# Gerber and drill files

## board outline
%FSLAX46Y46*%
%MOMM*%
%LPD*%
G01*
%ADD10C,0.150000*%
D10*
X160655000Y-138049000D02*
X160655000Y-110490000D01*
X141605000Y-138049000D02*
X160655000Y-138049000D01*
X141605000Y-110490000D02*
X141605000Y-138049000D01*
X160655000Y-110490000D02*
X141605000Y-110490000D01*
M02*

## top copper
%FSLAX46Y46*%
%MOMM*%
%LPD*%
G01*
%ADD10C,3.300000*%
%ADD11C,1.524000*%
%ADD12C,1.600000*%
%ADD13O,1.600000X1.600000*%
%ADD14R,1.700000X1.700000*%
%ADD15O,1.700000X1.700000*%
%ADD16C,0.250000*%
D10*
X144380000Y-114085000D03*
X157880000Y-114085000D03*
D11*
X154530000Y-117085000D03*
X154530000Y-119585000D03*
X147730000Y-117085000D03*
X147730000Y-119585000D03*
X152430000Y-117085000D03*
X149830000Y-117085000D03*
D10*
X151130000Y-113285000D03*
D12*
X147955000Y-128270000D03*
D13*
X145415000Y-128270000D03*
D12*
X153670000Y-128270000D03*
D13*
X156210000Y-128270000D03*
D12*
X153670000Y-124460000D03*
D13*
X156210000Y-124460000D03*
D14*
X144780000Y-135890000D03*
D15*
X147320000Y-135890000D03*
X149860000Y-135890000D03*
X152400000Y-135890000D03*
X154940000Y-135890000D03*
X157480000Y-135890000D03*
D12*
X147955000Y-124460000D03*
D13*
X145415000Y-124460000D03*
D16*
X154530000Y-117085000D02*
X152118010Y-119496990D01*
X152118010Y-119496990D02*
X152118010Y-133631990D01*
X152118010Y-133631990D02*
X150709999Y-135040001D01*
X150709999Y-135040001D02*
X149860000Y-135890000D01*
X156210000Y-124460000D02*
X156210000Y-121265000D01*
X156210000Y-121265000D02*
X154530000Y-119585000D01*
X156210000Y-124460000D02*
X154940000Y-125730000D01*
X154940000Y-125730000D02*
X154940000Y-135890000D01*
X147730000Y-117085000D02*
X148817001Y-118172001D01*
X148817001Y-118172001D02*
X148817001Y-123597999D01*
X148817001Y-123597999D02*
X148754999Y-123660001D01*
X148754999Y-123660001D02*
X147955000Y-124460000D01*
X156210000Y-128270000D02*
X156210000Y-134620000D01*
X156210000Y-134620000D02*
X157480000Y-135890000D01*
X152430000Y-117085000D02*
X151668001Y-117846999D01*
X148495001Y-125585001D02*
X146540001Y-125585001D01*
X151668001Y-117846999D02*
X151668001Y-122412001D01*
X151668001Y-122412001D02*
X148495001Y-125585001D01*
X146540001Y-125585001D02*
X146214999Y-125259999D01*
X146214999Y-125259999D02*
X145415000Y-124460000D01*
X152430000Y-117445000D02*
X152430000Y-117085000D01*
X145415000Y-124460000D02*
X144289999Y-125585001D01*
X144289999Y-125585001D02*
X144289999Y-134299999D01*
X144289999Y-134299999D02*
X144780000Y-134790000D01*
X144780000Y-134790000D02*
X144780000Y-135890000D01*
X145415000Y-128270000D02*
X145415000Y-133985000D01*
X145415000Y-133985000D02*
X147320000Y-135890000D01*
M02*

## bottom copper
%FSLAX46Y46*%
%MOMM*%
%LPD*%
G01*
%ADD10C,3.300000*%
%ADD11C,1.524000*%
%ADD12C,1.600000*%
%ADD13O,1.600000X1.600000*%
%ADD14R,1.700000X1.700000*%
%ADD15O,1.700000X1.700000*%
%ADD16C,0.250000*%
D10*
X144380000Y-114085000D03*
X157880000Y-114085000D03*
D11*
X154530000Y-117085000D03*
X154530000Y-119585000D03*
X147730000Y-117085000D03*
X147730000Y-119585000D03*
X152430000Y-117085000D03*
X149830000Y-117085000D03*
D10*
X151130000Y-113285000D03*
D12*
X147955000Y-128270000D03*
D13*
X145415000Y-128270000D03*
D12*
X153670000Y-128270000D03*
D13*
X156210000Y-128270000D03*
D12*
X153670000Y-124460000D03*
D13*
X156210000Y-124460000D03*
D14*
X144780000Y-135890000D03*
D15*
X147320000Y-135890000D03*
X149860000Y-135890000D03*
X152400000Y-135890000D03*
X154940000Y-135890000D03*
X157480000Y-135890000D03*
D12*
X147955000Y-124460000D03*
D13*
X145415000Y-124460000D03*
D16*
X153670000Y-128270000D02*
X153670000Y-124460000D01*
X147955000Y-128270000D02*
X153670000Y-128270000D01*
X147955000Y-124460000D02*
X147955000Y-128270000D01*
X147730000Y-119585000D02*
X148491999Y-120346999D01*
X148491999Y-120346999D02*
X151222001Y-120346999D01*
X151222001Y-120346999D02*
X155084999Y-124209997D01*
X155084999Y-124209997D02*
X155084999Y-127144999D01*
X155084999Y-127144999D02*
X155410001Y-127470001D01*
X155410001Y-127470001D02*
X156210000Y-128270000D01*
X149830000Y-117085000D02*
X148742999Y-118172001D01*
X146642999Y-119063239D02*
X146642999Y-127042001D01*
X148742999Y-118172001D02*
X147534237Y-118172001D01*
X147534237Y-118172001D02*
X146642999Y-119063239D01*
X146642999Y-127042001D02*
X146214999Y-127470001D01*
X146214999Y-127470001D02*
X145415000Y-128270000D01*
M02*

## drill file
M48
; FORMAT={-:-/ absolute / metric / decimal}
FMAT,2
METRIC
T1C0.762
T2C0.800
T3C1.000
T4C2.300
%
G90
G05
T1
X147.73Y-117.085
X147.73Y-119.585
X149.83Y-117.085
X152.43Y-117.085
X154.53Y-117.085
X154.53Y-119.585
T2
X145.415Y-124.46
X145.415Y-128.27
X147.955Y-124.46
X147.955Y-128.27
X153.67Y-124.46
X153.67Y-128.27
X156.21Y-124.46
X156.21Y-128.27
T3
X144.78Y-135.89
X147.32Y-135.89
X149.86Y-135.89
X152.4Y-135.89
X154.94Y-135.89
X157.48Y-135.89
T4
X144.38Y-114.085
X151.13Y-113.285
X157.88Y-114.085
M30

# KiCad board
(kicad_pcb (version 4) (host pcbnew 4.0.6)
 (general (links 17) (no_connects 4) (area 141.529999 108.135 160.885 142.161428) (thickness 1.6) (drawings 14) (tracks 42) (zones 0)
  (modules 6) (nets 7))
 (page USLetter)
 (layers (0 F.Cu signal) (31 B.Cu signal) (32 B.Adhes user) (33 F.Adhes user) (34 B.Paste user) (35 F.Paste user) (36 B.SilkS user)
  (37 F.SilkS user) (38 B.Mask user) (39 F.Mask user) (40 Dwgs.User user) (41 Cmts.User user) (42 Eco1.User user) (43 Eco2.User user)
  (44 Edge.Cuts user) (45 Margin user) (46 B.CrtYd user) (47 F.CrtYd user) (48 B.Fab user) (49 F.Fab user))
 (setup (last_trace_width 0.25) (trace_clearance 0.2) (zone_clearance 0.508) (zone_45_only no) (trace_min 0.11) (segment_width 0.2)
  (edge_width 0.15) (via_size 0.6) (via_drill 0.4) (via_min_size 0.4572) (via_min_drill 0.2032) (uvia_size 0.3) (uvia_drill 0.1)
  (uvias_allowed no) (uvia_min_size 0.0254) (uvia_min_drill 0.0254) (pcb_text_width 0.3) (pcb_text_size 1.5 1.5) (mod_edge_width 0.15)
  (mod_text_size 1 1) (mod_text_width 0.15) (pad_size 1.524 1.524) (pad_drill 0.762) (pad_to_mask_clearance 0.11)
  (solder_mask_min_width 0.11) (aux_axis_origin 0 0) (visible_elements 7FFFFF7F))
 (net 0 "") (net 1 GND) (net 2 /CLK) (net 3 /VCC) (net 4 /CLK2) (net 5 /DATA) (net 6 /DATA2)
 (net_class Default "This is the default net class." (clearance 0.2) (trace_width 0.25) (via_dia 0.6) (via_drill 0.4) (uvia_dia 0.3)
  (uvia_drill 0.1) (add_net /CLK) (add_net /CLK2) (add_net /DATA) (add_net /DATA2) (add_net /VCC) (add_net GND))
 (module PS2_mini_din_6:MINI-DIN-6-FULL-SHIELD (layer F.Cu) (at 151.13 108.585)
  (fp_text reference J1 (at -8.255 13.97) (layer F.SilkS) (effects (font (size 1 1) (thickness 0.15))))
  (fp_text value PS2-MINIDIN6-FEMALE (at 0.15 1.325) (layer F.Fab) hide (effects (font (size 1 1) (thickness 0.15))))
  (pad 7 thru_hole circle (at -6.75 5.5) (size 3.3 3.3) (drill 2.3) (layers *.Cu *.Mask) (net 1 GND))
  (pad 7 thru_hole circle (at 6.75 5.5) (size 3.3 3.3) (drill 2.3) (layers *.Cu *.Mask) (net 1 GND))
  (pad 3 thru_hole circle (at 3.4 8.5) (size 1.524 1.524) (drill 0.762) (layers *.Cu *.Mask) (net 1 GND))
  (pad 5 thru_hole circle (at 3.4 11) (size 1.524 1.524) (drill 0.762) (layers *.Cu *.Mask) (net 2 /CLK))
  (pad 4 thru_hole circle (at -3.4 8.5) (size 1.524 1.524) (drill 0.762) (layers *.Cu *.Mask) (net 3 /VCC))
  (pad 6 thru_hole circle (at -3.4 11) (size 1.524 1.524) (drill 0.762) (layers *.Cu *.Mask) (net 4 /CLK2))
  (pad 1 thru_hole circle (at 1.3 8.5) (size 1.524 1.524) (drill 0.762) (layers *.Cu *.Mask) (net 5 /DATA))
  (pad 2 thru_hole circle (at -1.3 8.5) (size 1.524 1.524) (drill 0.762) (layers *.Cu *.Mask) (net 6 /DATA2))
  (pad 7 thru_hole circle (at 0 4.7) (size 3.3 3.3) (drill 2.3) (layers *.Cu *.Mask) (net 1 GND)))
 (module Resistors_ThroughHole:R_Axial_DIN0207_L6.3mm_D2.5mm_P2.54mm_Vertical (layer F.Cu) (at 147.955 128.27 180)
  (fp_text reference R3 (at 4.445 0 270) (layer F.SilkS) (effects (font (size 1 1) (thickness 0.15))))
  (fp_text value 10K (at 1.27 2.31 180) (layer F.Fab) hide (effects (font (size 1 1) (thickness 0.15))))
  (pad 1 thru_hole circle (at 0 0 180) (size 1.6 1.6) (drill 0.8) (layers *.Cu *.Mask) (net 3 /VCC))
  (pad 2 thru_hole oval (at 2.54 0 180) (size 1.6 1.6) (drill 0.8) (layers *.Cu *.Mask) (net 6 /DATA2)))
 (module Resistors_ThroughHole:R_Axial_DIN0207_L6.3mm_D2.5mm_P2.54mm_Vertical (layer F.Cu) (at 153.67 128.27)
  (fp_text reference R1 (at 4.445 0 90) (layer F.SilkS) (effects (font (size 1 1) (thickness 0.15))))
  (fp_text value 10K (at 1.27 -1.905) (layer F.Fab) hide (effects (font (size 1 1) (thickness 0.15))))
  (pad 1 thru_hole circle (at 0 0) (size 1.6 1.6) (drill 0.8) (layers *.Cu *.Mask) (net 3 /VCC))
  (pad 2 thru_hole oval (at 2.54 0) (size 1.6 1.6) (drill 0.8) (layers *.Cu *.Mask) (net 4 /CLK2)))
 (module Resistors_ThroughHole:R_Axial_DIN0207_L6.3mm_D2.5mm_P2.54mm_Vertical (layer F.Cu) (at 153.67 124.46)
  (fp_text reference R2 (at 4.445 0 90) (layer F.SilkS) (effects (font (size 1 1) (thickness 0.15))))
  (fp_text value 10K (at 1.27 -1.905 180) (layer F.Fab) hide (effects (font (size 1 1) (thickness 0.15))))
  (pad 1 thru_hole circle (at 0 0) (size 1.6 1.6) (drill 0.8) (layers *.Cu *.Mask) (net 3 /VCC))
  (pad 2 thru_hole oval (at 2.54 0) (size 1.6 1.6) (drill 0.8) (layers *.Cu *.Mask) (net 2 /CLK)))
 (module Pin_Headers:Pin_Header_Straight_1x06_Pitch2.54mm (layer F.Cu) (at 144.78 135.89 90)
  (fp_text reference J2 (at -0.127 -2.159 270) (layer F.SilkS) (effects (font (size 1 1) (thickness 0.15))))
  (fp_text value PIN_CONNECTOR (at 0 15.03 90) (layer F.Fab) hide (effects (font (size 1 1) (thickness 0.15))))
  (pad 1 thru_hole rect (at 0 0 90) (size 1.7 1.7) (drill 1) (layers *.Cu *.Mask) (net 5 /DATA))
  (pad 2 thru_hole oval (at 0 2.54 90) (size 1.7 1.7) (drill 1) (layers *.Cu *.Mask) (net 6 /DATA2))
  (pad 3 thru_hole oval (at 0 5.08 90) (size 1.7 1.7) (drill 1) (layers *.Cu *.Mask) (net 1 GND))
  (pad 4 thru_hole oval (at 0 7.62 90) (size 1.7 1.7) (drill 1) (layers *.Cu *.Mask) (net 3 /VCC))
  (pad 5 thru_hole oval (at 0 10.16 90) (size 1.7 1.7) (drill 1) (layers *.Cu *.Mask) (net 2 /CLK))
  (pad 6 thru_hole oval (at 0 12.7 90) (size 1.7 1.7) (drill 1) (layers *.Cu *.Mask) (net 4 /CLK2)))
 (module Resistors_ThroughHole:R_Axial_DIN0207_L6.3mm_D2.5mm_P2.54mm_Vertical (layer F.Cu) (at 147.955 124.46 180)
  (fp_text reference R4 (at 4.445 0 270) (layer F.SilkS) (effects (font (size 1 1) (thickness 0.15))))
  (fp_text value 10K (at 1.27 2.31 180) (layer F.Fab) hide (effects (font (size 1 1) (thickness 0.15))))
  (pad 1 thru_hole circle (at 0 0 180) (size 1.6 1.6) (drill 0.8) (layers *.Cu *.Mask) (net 3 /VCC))
  (pad 2 thru_hole oval (at 2.54 0 180) (size 1.6 1.6) (drill 0.8) (layers *.Cu *.Mask) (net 5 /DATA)))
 (gr_line (start 160.655 138.049) (end 160.655 110.49) (layer Edge.Cuts) (width 0.15))
 (gr_line (start 141.605 138.049) (end 160.655 138.049) (layer Edge.Cuts) (width 0.15))
 (gr_line (start 141.605 110.49) (end 141.605 138.049) (layer Edge.Cuts) (width 0.15))
 (gr_line (start 160.655 110.49) (end 141.605 110.49) (layer Edge.Cuts) (width 0.15))
 (segment (start 154.53 117.085) (end 152.11801 119.49699) (width 0.25) (layer F.Cu) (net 1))
 (segment (start 152.11801 119.49699) (end 152.11801 133.63199) (width 0.25) (layer F.Cu) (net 1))
 (segment (start 152.11801 133.63199) (end 150.709999 135.040001) (width 0.25) (layer F.Cu) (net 1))
 (segment (start 150.709999 135.040001) (end 149.86 135.89) (width 0.25) (layer F.Cu) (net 1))
 (segment (start 156.21 124.46) (end 156.21 121.265) (width 0.25) (layer F.Cu) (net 2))
 (segment (start 156.21 121.265) (end 154.53 119.585) (width 0.25) (layer F.Cu) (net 2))
 (segment (start 156.21 124.46) (end 154.94 125.73) (width 0.25) (layer F.Cu) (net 2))
 (segment (start 154.94 125.73) (end 154.94 135.89) (width 0.25) (layer F.Cu) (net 2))
 (segment (start 153.67 128.27) (end 153.67 124.46) (width 0.25) (layer B.Cu) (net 3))
 (segment (start 147.955 128.27) (end 153.67 128.27) (width 0.25) (layer B.Cu) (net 3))
 (segment (start 147.955 124.46) (end 147.955 128.27) (width 0.25) (layer B.Cu) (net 3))
 (segment (start 147.73 117.085) (end 148.817001 118.172001) (width 0.25) (layer F.Cu) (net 3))
 (segment (start 148.817001 118.172001) (end 148.817001 123.597999) (width 0.25) (layer F.Cu) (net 3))
 (segment (start 148.817001 123.597999) (end 148.754999 123.660001) (width 0.25) (layer F.Cu) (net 3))
 (segment (start 148.754999 123.660001) (end 147.955 124.46) (width 0.25) (layer F.Cu) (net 3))
 (segment (start 147.73 119.585) (end 148.491999 120.346999) (width 0.25) (layer B.Cu) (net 4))
 (segment (start 148.491999 120.346999) (end 151.222001 120.346999) (width 0.25) (layer B.Cu) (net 4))
 (segment (start 151.222001 120.346999) (end 155.084999 124.209997) (width 0.25) (layer B.Cu) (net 4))
 (segment (start 155.084999 124.209997) (end 155.084999 127.144999) (width 0.25) (layer B.Cu) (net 4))
 (segment (start 155.084999 127.144999) (end 155.410001 127.470001) (width 0.25) (layer B.Cu) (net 4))
 (segment (start 155.410001 127.470001) (end 156.21 128.27) (width 0.25) (layer B.Cu) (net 4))
 (segment (start 156.21 128.27) (end 156.21 134.62) (width 0.25) (layer F.Cu) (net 4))
 (segment (start 156.21 134.62) (end 157.48 135.89) (width 0.25) (layer F.Cu) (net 4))
 (segment (start 152.43 117.085) (end 151.668001 117.846999) (width 0.25) (layer F.Cu) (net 5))
 (segment (start 148.495001 125.585001) (end 146.540001 125.585001) (width 0.25) (layer F.Cu) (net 5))
 (segment (start 151.668001 117.846999) (end 151.668001 122.412001) (width 0.25) (layer F.Cu) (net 5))
 (segment (start 151.668001 122.412001) (end 148.495001 125.585001) (width 0.25) (layer F.Cu) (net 5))
 (segment (start 146.540001 125.585001) (end 146.214999 125.259999) (width 0.25) (layer F.Cu) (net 5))
 (segment (start 146.214999 125.259999) (end 145.415 124.46) (width 0.25) (layer F.Cu) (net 5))
 (segment (start 152.43 117.445) (end 152.43 117.085) (width 0.25) (layer F.Cu) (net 5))
 (segment (start 145.415 124.46) (end 144.289999 125.585001) (width 0.25) (layer F.Cu) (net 5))
 (segment (start 144.289999 125.585001) (end 144.289999 134.299999) (width 0.25) (layer F.Cu) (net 5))
 (segment (start 144.289999 134.299999) (end 144.78 134.79) (width 0.25) (layer F.Cu) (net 5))
 (segment (start 144.78 134.79) (end 144.78 135.89) (width 0.25) (layer F.Cu) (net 5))
 (segment (start 149.83 117.085) (end 148.742999 118.172001) (width 0.25) (layer B.Cu) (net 6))
 (segment (start 146.642999 119.063239) (end 146.642999 127.042001) (width 0.25) (layer B.Cu) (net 6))
 (segment (start 148.742999 118.172001) (end 147.534237 118.172001) (width 0.25) (layer B.Cu) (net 6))
 (segment (start 147.534237 118.172001) (end 146.642999 119.063239) (width 0.25) (layer B.Cu) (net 6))
 (segment (start 146.642999 127.042001) (end 146.214999 127.470001) (width 0.25) (layer B.Cu) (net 6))
 (segment (start 146.214999 127.470001) (end 145.415 128.27) (width 0.25) (layer B.Cu) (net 6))
 (segment (start 145.415 128.27) (end 145.415 133.985) (width 0.25) (layer F.Cu) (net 6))
 (segment (start 145.415 133.985) (end 147.32 135.89) (width 0.25) (layer F.Cu) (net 6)))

